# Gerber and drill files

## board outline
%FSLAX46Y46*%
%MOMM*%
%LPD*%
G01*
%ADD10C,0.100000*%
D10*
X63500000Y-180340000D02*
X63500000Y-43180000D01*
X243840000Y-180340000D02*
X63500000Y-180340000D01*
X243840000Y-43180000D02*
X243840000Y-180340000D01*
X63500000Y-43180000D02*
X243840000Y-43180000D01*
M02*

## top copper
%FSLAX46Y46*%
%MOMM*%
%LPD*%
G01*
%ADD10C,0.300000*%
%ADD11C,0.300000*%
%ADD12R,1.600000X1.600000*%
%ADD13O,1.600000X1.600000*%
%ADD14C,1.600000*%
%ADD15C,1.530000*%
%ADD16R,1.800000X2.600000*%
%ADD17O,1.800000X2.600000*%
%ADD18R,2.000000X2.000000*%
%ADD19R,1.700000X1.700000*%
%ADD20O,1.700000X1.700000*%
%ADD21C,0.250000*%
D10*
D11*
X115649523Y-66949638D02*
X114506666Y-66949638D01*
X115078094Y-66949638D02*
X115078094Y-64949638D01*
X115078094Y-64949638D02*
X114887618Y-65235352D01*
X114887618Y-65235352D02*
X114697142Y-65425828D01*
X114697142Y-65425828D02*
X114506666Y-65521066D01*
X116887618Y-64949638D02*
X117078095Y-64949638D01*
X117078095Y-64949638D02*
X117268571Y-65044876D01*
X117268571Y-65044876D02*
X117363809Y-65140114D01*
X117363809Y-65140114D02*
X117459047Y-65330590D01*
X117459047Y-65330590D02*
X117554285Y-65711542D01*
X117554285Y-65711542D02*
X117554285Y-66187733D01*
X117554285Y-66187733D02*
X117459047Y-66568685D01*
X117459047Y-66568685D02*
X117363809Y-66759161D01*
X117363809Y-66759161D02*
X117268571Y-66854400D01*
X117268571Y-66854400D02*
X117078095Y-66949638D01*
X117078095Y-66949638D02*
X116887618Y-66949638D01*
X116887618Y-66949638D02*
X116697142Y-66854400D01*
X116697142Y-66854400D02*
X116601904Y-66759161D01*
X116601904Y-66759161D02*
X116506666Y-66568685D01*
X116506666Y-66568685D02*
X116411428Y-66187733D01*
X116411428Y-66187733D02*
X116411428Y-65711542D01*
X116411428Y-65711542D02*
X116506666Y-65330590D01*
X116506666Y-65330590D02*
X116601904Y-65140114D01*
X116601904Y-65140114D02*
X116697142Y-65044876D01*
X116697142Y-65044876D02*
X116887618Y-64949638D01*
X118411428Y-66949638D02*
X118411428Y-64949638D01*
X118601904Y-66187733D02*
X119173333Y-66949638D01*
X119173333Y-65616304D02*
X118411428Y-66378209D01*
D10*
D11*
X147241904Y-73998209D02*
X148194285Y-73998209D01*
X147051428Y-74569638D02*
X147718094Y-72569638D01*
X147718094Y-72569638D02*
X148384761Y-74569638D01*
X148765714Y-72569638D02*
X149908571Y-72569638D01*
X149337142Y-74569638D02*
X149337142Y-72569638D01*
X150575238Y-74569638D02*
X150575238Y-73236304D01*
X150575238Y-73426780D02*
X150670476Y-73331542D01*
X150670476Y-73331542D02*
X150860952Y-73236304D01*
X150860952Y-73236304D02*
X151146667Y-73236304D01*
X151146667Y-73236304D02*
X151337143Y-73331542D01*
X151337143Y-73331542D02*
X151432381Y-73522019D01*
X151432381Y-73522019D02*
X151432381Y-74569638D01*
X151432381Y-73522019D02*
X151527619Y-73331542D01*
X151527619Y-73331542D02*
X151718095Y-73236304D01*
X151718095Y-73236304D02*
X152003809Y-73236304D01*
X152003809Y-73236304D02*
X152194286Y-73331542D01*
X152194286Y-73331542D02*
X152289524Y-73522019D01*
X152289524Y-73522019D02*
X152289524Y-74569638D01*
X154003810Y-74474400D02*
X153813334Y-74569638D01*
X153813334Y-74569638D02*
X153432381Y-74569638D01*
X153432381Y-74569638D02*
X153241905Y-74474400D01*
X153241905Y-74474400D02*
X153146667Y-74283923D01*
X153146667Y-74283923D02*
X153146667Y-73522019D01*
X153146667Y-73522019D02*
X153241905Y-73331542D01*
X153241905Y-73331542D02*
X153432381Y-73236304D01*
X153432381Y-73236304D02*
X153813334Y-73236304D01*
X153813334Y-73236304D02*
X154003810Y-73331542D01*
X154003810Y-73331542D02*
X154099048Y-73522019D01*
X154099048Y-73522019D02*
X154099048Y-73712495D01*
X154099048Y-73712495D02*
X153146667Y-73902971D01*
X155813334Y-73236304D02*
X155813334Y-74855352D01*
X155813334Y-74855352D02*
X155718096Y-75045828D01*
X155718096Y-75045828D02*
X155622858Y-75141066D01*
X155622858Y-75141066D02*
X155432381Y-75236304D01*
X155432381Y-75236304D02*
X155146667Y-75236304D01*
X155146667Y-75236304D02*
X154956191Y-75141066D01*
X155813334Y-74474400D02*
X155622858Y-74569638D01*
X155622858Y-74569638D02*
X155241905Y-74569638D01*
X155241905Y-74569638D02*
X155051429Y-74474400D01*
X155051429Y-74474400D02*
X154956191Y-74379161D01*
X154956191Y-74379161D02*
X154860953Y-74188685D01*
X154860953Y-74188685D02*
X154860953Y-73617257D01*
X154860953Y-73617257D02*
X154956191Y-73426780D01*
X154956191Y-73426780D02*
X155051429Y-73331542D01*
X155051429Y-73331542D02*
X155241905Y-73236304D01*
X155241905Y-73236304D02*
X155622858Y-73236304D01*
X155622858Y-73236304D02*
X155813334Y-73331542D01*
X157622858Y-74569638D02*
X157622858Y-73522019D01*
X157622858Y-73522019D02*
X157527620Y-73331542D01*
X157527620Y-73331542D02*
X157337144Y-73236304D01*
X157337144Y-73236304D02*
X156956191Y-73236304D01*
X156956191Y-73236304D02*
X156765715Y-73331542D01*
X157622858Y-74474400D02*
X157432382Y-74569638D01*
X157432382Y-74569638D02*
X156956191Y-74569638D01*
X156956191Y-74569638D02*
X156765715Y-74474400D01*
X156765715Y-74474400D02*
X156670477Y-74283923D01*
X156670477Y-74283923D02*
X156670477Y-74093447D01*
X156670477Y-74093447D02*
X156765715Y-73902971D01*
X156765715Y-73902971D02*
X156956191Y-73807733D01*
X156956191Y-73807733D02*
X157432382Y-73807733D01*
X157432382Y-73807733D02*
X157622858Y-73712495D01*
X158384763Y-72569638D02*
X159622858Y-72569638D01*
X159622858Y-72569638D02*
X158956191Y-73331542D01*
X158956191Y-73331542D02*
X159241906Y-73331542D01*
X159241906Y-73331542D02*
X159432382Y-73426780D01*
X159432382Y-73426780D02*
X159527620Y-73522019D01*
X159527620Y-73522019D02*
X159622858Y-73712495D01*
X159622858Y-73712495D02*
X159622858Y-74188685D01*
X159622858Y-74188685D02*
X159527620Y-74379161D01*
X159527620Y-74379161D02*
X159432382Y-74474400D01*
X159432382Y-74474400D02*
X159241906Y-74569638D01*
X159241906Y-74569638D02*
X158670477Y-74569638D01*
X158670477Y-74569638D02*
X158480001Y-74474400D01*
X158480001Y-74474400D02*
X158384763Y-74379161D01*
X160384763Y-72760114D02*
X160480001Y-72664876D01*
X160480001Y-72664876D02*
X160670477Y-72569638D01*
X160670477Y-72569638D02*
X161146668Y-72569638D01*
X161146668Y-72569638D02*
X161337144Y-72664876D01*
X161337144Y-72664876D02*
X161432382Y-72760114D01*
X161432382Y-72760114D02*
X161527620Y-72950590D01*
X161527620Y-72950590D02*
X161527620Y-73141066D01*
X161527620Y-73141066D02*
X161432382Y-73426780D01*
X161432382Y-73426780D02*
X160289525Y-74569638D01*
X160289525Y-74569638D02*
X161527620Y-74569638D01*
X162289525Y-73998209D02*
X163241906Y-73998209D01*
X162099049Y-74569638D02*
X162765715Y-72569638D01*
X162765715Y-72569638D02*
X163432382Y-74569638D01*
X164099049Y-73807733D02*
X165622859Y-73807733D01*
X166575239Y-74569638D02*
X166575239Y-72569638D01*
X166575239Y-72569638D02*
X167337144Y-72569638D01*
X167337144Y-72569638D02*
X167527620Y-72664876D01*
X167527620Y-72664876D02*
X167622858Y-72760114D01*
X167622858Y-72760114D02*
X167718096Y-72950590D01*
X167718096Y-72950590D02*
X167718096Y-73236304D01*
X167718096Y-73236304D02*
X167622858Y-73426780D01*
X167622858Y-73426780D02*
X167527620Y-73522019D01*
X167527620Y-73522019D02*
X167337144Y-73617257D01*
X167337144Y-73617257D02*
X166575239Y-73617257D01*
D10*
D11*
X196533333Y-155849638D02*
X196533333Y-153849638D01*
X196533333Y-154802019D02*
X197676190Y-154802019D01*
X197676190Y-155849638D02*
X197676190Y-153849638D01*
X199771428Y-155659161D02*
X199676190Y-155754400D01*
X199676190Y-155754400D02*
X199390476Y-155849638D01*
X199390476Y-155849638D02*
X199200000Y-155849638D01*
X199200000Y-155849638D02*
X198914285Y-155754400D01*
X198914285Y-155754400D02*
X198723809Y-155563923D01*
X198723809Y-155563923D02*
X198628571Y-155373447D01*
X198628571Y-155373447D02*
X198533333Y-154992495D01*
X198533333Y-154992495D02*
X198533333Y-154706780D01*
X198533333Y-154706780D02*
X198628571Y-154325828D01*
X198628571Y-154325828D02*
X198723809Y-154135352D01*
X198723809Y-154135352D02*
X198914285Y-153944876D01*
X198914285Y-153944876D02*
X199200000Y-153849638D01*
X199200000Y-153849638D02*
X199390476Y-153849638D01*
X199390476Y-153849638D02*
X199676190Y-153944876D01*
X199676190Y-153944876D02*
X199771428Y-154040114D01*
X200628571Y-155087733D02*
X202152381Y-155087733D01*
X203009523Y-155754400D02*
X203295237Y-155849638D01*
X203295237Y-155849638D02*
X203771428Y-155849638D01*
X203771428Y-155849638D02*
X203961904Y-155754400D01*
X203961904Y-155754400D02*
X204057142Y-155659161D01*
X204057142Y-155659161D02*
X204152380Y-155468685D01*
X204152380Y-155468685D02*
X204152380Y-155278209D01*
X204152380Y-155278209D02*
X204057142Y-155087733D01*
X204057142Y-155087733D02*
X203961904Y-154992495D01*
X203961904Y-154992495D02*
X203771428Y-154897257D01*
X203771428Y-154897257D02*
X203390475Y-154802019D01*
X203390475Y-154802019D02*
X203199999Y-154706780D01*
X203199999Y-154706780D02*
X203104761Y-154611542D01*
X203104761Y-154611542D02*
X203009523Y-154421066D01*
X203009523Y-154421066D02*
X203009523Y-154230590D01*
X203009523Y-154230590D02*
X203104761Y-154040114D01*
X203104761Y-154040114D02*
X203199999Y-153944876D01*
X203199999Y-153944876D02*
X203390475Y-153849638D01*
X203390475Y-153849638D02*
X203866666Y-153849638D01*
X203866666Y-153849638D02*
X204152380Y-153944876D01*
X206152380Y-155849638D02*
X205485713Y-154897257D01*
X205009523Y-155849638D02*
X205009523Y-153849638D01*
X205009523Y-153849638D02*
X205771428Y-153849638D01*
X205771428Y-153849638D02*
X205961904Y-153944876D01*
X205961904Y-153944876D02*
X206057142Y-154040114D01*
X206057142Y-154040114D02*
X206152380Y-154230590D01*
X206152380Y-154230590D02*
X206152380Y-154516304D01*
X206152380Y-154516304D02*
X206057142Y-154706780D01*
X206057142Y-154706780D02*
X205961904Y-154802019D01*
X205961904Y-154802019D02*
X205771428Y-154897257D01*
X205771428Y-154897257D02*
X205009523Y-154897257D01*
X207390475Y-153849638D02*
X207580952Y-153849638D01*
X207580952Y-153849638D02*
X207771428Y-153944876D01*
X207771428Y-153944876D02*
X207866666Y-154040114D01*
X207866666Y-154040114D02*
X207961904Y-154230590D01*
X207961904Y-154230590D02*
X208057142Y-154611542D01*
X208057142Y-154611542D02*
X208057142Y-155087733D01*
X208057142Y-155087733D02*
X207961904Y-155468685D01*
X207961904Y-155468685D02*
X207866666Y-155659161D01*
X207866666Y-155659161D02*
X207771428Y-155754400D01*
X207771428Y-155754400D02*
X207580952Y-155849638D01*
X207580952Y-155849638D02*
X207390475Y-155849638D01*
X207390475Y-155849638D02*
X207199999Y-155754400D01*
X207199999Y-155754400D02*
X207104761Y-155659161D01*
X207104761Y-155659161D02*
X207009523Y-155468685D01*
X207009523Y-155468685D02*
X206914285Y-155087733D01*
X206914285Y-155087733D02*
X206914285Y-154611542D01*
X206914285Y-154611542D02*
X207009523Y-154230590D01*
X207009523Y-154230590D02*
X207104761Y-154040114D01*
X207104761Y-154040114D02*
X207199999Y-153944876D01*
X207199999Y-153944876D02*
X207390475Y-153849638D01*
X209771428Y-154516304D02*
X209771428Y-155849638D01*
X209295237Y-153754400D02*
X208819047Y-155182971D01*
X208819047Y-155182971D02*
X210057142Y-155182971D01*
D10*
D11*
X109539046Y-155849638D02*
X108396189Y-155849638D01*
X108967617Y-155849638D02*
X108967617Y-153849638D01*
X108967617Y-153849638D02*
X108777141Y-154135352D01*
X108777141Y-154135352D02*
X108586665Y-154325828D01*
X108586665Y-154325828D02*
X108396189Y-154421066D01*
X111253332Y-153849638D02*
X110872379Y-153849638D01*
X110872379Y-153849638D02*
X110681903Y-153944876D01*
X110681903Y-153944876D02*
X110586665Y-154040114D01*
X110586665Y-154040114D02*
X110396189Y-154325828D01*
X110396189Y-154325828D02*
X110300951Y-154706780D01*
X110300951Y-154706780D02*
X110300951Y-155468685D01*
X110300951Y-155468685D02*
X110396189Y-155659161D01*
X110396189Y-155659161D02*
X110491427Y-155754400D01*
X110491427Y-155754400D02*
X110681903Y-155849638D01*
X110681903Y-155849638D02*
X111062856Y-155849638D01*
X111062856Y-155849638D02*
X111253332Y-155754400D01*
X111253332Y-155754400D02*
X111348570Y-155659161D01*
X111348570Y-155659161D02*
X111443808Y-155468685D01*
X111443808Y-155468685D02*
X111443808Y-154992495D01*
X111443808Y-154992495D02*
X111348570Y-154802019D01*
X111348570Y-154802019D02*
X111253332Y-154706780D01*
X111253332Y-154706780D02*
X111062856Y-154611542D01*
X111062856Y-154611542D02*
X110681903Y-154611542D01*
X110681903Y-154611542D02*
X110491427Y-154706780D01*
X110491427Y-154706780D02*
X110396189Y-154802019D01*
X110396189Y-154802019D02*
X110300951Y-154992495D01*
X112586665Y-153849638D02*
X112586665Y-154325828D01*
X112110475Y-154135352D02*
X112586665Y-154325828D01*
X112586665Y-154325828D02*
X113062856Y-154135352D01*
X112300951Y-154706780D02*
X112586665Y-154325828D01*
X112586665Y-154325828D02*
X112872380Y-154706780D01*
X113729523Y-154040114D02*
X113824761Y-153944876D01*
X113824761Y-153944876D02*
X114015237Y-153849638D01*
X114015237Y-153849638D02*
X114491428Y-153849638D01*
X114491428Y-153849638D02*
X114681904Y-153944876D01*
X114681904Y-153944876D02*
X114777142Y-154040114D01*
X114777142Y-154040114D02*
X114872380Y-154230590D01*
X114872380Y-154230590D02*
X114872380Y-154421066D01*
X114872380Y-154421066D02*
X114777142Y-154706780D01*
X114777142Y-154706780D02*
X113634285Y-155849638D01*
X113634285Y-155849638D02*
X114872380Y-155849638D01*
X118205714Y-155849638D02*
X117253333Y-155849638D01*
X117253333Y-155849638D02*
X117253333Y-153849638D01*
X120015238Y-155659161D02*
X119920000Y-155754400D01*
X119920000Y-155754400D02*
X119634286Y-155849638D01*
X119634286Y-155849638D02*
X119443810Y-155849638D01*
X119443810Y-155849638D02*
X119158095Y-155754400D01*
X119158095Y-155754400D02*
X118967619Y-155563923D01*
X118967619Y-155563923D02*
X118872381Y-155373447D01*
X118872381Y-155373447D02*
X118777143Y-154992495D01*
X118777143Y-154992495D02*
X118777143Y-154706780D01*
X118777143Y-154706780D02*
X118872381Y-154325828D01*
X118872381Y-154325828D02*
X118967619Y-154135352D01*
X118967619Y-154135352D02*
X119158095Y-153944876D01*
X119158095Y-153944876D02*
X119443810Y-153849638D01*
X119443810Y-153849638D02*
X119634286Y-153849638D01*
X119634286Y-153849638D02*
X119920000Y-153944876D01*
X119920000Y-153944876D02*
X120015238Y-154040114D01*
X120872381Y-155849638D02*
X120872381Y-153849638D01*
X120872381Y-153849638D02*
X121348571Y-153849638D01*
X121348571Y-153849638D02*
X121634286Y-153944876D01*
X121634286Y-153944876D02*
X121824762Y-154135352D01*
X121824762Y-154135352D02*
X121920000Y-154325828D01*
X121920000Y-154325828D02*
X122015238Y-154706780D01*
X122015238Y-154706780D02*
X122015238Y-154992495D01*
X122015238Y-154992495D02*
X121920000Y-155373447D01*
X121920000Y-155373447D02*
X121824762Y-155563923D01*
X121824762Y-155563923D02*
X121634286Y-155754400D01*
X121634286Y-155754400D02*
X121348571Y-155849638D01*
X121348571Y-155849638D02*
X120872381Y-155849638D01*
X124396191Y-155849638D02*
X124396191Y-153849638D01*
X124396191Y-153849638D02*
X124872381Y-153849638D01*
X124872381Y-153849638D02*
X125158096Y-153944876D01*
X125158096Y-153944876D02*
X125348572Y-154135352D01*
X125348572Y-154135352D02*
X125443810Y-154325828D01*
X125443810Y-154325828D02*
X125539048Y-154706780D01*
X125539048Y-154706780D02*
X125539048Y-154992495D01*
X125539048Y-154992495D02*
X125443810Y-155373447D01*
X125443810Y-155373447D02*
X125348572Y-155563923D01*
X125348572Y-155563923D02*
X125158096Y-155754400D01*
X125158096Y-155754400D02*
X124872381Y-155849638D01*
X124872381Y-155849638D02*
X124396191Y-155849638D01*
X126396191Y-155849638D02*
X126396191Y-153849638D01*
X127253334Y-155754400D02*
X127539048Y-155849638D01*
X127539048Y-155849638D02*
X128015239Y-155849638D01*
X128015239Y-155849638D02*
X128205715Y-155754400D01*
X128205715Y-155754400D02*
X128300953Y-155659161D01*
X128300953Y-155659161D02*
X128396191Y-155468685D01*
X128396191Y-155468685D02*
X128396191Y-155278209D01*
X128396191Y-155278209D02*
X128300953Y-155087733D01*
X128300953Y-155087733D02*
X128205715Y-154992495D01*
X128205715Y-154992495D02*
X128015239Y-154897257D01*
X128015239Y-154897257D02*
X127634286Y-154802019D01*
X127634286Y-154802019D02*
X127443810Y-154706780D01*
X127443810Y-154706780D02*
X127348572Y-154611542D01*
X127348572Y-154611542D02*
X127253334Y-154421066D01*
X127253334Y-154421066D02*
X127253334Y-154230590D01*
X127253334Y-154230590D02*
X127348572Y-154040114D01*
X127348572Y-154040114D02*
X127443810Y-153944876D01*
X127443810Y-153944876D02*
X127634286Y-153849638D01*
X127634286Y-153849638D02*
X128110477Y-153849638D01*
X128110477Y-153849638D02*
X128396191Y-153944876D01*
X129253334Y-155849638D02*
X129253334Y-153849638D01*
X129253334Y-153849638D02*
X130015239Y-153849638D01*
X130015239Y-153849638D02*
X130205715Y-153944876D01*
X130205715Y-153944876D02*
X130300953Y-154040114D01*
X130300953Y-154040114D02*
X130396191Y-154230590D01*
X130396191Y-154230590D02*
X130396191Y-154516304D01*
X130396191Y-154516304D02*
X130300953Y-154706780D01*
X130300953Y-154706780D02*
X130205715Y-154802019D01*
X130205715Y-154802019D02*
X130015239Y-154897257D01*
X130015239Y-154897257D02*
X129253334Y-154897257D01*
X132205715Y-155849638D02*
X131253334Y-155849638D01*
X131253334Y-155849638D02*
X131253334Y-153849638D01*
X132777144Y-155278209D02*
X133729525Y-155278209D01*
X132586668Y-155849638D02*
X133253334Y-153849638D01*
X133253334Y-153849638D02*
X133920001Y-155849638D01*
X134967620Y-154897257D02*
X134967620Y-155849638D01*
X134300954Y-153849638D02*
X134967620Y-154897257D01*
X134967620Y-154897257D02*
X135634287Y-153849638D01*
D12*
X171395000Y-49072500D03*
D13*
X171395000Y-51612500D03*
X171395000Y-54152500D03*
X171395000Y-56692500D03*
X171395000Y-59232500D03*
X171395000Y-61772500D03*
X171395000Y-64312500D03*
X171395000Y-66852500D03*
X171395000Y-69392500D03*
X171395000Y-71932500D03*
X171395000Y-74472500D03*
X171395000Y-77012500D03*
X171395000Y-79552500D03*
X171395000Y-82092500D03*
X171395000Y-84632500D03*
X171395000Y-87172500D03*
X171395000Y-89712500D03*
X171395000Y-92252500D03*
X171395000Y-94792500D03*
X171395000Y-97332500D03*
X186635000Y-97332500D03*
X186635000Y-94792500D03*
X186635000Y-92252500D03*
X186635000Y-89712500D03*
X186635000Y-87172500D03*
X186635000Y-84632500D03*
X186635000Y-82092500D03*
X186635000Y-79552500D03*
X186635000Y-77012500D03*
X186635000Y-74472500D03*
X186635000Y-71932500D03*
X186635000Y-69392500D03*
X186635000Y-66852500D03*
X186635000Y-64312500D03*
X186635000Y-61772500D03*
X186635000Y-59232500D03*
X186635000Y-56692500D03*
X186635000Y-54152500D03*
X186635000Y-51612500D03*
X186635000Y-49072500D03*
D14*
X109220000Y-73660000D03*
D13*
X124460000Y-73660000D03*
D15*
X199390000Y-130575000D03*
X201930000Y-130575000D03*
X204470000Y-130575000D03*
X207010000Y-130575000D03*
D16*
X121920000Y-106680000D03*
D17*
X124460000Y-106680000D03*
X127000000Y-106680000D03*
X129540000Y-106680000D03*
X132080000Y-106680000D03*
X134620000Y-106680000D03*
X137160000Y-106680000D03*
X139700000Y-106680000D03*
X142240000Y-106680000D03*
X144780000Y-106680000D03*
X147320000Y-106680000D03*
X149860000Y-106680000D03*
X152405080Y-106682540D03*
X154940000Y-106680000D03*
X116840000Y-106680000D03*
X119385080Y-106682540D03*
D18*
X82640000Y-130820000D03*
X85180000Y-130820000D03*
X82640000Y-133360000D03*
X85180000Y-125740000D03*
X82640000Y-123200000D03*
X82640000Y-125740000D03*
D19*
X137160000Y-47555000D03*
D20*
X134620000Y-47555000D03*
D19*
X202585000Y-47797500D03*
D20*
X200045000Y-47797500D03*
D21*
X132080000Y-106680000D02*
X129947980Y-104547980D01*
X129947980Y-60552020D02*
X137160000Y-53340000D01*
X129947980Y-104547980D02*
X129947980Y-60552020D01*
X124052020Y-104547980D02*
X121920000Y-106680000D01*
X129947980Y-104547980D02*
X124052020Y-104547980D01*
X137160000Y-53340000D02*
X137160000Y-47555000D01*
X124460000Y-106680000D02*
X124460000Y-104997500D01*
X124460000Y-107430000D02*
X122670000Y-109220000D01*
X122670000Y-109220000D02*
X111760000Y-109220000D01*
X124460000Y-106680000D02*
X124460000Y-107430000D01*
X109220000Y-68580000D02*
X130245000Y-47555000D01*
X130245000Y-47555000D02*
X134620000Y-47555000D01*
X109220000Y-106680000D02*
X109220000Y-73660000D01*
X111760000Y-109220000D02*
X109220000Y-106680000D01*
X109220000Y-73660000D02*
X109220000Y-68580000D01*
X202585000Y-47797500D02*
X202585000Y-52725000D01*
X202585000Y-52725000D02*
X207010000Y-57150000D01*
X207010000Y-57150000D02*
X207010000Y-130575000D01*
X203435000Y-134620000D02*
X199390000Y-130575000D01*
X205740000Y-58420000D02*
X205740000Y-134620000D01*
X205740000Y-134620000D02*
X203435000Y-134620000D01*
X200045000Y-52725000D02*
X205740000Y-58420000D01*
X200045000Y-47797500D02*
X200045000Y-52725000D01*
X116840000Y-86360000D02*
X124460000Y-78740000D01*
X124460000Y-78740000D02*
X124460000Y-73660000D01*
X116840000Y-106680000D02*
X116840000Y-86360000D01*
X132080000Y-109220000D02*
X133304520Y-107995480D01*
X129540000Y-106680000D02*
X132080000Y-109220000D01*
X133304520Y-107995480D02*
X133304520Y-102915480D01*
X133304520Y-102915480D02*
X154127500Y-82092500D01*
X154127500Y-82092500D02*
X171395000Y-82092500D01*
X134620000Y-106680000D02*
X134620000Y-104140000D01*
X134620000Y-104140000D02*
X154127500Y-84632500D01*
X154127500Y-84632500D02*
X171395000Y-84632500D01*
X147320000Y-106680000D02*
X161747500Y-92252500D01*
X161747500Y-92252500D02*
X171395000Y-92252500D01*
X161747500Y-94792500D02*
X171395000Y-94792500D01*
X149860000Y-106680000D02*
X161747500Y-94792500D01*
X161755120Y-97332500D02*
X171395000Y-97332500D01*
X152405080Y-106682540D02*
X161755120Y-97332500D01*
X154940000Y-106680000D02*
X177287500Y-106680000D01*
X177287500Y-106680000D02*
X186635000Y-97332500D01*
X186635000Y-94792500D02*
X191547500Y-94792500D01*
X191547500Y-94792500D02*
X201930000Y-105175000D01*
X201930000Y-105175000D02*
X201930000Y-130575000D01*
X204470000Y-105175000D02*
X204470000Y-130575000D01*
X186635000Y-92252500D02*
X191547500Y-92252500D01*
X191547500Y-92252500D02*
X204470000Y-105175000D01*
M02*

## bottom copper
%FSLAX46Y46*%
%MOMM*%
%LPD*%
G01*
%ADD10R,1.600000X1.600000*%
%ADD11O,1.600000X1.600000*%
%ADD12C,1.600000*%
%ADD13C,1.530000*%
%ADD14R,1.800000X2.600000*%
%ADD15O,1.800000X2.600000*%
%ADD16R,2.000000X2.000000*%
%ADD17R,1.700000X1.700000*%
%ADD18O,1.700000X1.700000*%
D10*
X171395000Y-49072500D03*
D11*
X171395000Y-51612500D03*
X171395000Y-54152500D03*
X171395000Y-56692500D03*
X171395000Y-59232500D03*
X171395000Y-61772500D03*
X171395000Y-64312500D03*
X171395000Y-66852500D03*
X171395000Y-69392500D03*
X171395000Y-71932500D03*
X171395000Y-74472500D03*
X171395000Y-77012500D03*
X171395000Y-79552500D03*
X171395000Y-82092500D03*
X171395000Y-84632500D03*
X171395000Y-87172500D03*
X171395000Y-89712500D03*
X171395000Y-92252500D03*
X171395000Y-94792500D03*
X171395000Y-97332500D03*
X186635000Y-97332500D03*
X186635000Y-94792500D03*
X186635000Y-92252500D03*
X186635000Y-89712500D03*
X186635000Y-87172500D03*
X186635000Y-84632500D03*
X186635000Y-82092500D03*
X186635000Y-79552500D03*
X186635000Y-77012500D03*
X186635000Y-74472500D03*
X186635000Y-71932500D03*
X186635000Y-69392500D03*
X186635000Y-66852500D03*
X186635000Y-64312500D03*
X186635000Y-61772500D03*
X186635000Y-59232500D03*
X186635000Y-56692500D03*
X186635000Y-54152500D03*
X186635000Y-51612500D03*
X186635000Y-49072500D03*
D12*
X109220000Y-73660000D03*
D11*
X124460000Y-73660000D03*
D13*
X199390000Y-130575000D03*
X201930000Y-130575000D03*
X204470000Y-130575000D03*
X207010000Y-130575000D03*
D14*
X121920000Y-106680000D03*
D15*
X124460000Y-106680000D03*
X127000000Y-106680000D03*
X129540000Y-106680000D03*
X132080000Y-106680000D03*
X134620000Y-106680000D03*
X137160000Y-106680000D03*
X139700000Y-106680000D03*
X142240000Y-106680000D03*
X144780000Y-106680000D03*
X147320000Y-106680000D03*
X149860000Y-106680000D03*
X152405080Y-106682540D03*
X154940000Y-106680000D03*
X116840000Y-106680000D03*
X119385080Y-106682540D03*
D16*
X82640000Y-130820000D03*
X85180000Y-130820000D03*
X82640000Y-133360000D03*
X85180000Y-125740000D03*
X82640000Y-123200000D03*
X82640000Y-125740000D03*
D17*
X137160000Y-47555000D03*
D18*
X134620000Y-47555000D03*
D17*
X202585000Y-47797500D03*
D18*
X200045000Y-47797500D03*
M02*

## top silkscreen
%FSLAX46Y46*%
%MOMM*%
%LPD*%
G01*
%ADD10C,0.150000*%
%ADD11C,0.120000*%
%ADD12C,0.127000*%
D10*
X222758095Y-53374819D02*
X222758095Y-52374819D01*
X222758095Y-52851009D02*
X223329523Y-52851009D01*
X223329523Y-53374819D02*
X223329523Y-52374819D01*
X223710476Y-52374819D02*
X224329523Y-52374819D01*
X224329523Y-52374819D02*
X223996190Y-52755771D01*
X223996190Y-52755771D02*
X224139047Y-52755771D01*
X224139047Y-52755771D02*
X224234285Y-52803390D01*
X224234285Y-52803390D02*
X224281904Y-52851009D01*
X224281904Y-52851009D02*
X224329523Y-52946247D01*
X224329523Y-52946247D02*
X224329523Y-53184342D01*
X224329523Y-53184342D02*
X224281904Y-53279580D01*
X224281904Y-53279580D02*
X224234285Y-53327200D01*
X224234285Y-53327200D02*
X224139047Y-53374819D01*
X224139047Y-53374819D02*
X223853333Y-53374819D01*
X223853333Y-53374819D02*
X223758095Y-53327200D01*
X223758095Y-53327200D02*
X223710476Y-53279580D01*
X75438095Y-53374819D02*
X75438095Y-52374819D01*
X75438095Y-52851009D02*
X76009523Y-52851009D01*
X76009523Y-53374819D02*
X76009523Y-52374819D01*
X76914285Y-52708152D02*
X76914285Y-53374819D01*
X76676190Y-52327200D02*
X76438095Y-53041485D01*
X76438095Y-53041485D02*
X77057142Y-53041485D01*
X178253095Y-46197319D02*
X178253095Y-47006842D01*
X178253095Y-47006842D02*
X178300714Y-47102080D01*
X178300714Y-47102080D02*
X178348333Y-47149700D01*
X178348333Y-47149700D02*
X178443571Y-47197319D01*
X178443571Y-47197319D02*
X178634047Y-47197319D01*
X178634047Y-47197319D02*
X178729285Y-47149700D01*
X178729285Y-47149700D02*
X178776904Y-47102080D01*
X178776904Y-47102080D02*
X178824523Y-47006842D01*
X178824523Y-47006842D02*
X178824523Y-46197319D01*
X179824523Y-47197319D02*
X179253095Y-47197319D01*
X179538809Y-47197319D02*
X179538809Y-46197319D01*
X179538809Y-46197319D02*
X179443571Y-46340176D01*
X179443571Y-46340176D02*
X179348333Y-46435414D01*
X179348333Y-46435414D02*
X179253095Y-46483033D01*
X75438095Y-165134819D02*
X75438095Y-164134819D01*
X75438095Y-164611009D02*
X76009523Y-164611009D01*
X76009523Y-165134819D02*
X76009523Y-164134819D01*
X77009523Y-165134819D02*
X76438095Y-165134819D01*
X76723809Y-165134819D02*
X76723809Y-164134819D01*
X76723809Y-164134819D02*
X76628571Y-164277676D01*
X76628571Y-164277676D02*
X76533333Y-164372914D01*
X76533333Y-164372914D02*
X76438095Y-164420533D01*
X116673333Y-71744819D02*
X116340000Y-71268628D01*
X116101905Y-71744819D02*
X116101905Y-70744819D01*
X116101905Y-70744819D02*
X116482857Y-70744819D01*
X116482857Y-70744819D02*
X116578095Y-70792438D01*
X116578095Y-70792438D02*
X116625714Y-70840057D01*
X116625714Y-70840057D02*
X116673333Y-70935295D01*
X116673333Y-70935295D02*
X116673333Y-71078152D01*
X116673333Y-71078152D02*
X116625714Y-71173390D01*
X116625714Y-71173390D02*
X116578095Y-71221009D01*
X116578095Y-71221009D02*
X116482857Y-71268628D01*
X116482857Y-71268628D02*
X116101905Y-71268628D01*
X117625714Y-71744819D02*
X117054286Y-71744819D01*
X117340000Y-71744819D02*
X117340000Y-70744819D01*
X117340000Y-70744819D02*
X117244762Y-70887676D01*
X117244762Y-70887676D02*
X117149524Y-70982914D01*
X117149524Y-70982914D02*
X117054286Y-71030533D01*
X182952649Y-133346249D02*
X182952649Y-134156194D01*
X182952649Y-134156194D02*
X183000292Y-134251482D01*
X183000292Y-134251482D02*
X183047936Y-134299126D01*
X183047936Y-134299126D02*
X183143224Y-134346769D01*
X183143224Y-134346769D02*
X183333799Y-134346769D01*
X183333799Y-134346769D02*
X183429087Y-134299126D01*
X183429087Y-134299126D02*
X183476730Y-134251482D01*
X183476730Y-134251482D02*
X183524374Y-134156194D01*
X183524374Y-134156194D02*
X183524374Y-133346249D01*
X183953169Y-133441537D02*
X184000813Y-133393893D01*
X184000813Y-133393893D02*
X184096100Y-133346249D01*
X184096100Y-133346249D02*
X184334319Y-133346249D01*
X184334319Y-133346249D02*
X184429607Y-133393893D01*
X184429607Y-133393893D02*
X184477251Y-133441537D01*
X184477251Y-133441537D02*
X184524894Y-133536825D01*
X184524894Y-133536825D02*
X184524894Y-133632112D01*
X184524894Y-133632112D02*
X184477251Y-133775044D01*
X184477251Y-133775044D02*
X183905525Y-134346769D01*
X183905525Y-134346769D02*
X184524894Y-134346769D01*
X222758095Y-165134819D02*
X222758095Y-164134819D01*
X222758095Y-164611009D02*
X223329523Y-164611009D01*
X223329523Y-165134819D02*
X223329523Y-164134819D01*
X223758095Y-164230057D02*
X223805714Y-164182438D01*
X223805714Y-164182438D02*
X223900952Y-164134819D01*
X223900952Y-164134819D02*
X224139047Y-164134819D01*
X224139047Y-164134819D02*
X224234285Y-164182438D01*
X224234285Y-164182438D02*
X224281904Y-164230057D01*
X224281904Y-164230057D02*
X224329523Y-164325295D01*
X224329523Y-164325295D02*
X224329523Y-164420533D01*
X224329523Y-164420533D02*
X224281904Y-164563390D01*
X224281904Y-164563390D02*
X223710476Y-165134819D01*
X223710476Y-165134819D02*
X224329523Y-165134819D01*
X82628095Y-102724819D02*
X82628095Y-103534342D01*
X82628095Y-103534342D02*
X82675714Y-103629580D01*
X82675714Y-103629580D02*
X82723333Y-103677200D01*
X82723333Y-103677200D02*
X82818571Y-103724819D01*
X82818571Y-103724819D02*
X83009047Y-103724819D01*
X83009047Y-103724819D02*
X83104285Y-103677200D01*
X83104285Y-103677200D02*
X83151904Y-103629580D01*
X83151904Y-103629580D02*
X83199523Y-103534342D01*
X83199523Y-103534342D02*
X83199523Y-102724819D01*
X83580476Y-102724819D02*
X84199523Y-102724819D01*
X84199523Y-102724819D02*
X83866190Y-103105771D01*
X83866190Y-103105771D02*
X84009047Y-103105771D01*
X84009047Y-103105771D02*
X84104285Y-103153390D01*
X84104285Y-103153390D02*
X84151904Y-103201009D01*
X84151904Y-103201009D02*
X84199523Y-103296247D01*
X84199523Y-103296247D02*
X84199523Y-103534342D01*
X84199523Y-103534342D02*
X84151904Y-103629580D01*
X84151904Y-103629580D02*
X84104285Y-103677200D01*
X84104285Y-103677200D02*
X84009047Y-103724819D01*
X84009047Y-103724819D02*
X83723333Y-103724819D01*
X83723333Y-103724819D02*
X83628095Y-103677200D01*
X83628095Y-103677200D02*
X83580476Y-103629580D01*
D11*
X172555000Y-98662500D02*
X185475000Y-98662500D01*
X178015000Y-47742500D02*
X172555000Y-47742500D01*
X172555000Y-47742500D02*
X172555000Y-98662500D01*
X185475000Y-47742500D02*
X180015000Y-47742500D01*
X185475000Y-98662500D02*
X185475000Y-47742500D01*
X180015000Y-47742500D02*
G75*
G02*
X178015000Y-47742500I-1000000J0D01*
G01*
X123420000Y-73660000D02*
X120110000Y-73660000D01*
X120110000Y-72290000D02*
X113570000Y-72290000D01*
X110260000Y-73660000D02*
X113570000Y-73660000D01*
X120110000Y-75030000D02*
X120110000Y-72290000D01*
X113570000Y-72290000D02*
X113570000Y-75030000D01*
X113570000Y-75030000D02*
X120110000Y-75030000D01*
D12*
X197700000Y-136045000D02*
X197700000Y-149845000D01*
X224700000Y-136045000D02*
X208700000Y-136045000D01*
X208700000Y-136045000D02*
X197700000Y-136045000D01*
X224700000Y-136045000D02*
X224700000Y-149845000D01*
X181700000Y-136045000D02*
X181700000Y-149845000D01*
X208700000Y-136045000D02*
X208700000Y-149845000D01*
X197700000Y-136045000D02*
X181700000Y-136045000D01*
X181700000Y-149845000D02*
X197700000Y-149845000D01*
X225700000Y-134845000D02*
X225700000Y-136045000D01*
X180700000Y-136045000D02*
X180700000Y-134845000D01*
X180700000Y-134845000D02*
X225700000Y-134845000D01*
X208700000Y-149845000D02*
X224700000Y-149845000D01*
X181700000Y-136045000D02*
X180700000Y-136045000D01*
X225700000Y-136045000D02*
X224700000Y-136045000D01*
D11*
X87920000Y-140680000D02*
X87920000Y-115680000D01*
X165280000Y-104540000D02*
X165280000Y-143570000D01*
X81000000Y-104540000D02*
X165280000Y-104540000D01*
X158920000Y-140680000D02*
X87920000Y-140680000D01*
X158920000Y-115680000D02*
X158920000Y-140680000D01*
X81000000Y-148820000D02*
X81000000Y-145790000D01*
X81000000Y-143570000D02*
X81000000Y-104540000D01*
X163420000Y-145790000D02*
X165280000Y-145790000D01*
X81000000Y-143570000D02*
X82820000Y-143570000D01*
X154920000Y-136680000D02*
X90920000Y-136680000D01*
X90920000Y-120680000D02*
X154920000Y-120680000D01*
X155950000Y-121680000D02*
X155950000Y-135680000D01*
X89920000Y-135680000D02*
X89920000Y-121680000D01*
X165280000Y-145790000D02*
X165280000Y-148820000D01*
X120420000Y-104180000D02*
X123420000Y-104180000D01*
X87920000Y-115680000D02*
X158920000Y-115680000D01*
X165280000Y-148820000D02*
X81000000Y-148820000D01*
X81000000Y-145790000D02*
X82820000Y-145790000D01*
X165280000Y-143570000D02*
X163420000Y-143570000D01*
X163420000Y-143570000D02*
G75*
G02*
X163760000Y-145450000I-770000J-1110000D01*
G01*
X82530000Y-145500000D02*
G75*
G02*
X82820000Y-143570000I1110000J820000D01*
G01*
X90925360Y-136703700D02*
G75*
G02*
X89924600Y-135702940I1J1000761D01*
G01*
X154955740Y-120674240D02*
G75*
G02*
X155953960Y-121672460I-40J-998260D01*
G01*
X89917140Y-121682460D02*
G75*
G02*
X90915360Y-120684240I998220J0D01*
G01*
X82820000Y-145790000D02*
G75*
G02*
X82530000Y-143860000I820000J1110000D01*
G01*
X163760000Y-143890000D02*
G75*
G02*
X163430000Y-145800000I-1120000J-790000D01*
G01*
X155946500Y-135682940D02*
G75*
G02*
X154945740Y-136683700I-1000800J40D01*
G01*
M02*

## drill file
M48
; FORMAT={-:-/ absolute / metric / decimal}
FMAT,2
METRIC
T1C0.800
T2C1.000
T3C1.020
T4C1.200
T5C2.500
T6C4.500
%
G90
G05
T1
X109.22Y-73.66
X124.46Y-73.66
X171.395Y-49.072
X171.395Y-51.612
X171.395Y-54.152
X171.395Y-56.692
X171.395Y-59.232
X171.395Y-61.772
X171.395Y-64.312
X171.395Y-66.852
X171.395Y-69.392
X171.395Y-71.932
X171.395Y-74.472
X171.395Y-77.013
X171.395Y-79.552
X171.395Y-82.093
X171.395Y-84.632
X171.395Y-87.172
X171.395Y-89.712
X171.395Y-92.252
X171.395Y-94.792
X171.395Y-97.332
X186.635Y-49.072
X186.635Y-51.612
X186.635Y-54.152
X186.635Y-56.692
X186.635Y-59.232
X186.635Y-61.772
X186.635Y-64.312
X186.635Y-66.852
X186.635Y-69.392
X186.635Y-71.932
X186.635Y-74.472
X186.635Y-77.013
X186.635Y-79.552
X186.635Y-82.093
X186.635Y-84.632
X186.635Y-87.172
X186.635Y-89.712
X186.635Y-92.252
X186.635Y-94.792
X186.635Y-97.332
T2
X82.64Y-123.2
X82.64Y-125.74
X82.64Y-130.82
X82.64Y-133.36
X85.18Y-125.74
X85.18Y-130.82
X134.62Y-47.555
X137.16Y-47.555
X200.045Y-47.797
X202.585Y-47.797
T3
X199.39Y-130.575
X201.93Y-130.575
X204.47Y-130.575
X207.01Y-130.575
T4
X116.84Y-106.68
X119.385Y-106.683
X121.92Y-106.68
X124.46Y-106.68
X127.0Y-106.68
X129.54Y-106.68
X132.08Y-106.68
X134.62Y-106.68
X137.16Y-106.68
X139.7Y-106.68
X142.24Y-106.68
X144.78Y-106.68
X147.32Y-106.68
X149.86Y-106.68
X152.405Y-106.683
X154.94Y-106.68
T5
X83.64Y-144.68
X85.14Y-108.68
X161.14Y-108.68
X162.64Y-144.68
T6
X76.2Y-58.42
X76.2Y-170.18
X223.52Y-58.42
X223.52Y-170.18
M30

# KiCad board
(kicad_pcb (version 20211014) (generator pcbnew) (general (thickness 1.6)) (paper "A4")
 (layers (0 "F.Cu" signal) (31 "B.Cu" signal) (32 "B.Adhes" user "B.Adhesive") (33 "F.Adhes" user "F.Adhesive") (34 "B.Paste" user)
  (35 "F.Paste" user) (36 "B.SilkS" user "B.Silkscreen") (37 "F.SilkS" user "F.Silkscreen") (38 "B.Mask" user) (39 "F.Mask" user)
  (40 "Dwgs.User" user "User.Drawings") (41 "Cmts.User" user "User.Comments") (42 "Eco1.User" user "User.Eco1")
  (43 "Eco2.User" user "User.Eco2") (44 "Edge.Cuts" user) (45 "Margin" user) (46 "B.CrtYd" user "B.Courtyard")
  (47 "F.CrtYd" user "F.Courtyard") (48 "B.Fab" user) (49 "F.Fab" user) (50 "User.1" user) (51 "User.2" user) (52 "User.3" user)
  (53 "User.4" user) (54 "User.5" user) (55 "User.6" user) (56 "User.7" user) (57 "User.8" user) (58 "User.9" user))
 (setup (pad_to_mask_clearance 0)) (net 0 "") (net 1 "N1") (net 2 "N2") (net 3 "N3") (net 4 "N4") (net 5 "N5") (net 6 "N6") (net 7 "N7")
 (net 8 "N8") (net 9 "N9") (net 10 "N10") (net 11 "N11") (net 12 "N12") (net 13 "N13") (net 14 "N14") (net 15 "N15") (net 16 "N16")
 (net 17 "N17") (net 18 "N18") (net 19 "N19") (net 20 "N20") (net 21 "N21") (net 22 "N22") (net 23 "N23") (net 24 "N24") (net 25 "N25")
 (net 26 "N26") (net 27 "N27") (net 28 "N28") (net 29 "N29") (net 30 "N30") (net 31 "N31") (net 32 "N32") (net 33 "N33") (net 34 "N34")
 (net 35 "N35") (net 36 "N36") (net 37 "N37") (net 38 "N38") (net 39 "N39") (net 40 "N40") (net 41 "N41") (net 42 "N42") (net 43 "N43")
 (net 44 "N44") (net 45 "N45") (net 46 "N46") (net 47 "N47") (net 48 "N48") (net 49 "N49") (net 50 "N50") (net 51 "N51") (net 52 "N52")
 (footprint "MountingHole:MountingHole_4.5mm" (layer "F.Cu") (at 223.52 58.42)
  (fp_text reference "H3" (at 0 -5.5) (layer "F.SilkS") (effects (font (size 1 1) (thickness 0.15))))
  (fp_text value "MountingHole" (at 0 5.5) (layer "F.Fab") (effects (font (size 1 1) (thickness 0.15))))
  (pad "" np_thru_hole circle (at 0 0) (size 4.5 4.5) (drill 4.5) (layers *.Cu *.Mask)))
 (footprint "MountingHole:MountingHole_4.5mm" (layer "F.Cu") (at 76.2 58.42)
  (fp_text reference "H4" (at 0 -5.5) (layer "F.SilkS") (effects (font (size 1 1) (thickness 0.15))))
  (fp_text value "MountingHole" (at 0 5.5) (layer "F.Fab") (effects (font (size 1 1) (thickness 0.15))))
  (pad "" np_thru_hole circle (at 0 0) (size 4.5 4.5) (drill 4.5) (layers *.Cu *.Mask)))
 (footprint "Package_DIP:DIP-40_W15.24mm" (layer "F.Cu") (at 171.395 49.0725)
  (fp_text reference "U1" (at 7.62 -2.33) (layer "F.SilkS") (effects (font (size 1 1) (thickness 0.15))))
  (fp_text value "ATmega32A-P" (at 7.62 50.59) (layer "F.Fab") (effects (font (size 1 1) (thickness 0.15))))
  (fp_line (start 1.16 49.59) (end 14.08 49.59) (layer "F.SilkS") (width 0.12))
  (fp_line (start 6.62 -1.33) (end 1.16 -1.33) (layer "F.SilkS") (width 0.12))
  (fp_line (start 1.16 -1.33) (end 1.16 49.59) (layer "F.SilkS") (width 0.12))
  (fp_line (start 14.08 -1.33) (end 8.62 -1.33) (layer "F.SilkS") (width 0.12))
  (fp_line (start 14.08 49.59) (end 14.08 -1.33) (layer "F.SilkS") (width 0.12))
  (fp_arc (start 8.62 -1.33) (mid 7.62 -0.33) (end 6.62 -1.33) (layer "F.SilkS") (width 0.12))
  (pad "1" thru_hole rect (at 0 0) (size 1.6 1.6) (drill 0.8) (layers *.Cu *.Mask) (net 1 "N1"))
  (pad "2" thru_hole oval (at 0 2.54) (size 1.6 1.6) (drill 0.8) (layers *.Cu *.Mask) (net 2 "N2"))
  (pad "3" thru_hole oval (at 0 5.08) (size 1.6 1.6) (drill 0.8) (layers *.Cu *.Mask) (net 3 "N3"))
  (pad "4" thru_hole oval (at 0 7.62) (size 1.6 1.6) (drill 0.8) (layers *.Cu *.Mask) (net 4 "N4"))
  (pad "5" thru_hole oval (at 0 10.16) (size 1.6 1.6) (drill 0.8) (layers *.Cu *.Mask) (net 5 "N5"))
  (pad "6" thru_hole oval (at 0 12.7) (size 1.6 1.6) (drill 0.8) (layers *.Cu *.Mask) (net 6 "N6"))
  (pad "7" thru_hole oval (at 0 15.24) (size 1.6 1.6) (drill 0.8) (layers *.Cu *.Mask) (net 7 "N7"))
  (pad "8" thru_hole oval (at 0 17.78) (size 1.6 1.6) (drill 0.8) (layers *.Cu *.Mask) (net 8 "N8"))
  (pad "9" thru_hole oval (at 0 20.32) (size 1.6 1.6) (drill 0.8) (layers *.Cu *.Mask) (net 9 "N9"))
  (pad "10" thru_hole oval (at 0 22.86) (size 1.6 1.6) (drill 0.8) (layers *.Cu *.Mask) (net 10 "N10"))
  (pad "11" thru_hole oval (at 0 25.4) (size 1.6 1.6) (drill 0.8) (layers *.Cu *.Mask) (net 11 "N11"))
  (pad "12" thru_hole oval (at 0 27.94) (size 1.6 1.6) (drill 0.8) (layers *.Cu *.Mask) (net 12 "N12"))
  (pad "13" thru_hole oval (at 0 30.48) (size 1.6 1.6) (drill 0.8) (layers *.Cu *.Mask) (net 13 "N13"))
  (pad "14" thru_hole oval (at 0 33.02) (size 1.6 1.6) (drill 0.8) (layers *.Cu *.Mask) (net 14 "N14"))
  (pad "15" thru_hole oval (at 0 35.56) (size 1.6 1.6) (drill 0.8) (layers *.Cu *.Mask) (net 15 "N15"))
  (pad "16" thru_hole oval (at 0 38.1) (size 1.6 1.6) (drill 0.8) (layers *.Cu *.Mask) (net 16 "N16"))
  (pad "17" thru_hole oval (at 0 40.64) (size 1.6 1.6) (drill 0.8) (layers *.Cu *.Mask) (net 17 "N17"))
  (pad "18" thru_hole oval (at 0 43.18) (size 1.6 1.6) (drill 0.8) (layers *.Cu *.Mask) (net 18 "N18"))
  (pad "19" thru_hole oval (at 0 45.72) (size 1.6 1.6) (drill 0.8) (layers *.Cu *.Mask) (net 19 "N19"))
  (pad "20" thru_hole oval (at 0 48.26) (size 1.6 1.6) (drill 0.8) (layers *.Cu *.Mask) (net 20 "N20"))
  (pad "21" thru_hole oval (at 15.24 48.26) (size 1.6 1.6) (drill 0.8) (layers *.Cu *.Mask) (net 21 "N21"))
  (pad "22" thru_hole oval (at 15.24 45.72) (size 1.6 1.6) (drill 0.8) (layers *.Cu *.Mask) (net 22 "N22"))
  (pad "23" thru_hole oval (at 15.24 43.18) (size 1.6 1.6) (drill 0.8) (layers *.Cu *.Mask) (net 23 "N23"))
  (pad "24" thru_hole oval (at 15.24 40.64) (size 1.6 1.6) (drill 0.8) (layers *.Cu *.Mask) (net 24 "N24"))
  (pad "25" thru_hole oval (at 15.24 38.1) (size 1.6 1.6) (drill 0.8) (layers *.Cu *.Mask) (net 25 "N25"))
  (pad "26" thru_hole oval (at 15.24 35.56) (size 1.6 1.6) (drill 0.8) (layers *.Cu *.Mask) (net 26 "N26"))
  (pad "27" thru_hole oval (at 15.24 33.02) (size 1.6 1.6) (drill 0.8) (layers *.Cu *.Mask) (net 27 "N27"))
  (pad "28" thru_hole oval (at 15.24 30.48) (size 1.6 1.6) (drill 0.8) (layers *.Cu *.Mask) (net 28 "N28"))
  (pad "29" thru_hole oval (at 15.24 27.94) (size 1.6 1.6) (drill 0.8) (layers *.Cu *.Mask) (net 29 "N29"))
  (pad "30" thru_hole oval (at 15.24 25.4) (size 1.6 1.6) (drill 0.8) (layers *.Cu *.Mask) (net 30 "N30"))
  (pad "31" thru_hole oval (at 15.24 22.86) (size 1.6 1.6) (drill 0.8) (layers *.Cu *.Mask) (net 11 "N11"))
  (pad "32" thru_hole oval (at 15.24 20.32) (size 1.6 1.6) (drill 0.8) (layers *.Cu *.Mask) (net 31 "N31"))
  (pad "33" thru_hole oval (at 15.24 17.78) (size 1.6 1.6) (drill 0.8) (layers *.Cu *.Mask) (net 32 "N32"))
  (pad "34" thru_hole oval (at 15.24 15.24) (size 1.6 1.6) (drill 0.8) (layers *.Cu *.Mask) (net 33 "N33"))
  (pad "35" thru_hole oval (at 15.24 12.7) (size 1.6 1.6) (drill 0.8) (layers *.Cu *.Mask) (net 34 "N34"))
  (pad "36" thru_hole oval (at 15.24 10.16) (size 1.6 1.6) (drill 0.8) (layers *.Cu *.Mask) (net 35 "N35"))
  (pad "37" thru_hole oval (at 15.24 7.62) (size 1.6 1.6) (drill 0.8) (layers *.Cu *.Mask) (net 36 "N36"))
  (pad "38" thru_hole oval (at 15.24 5.08) (size 1.6 1.6) (drill 0.8) (layers *.Cu *.Mask) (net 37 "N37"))
  (pad "39" thru_hole oval (at 15.24 2.54) (size 1.6 1.6) (drill 0.8) (layers *.Cu *.Mask) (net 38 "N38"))
  (pad "40" thru_hole oval (at 15.24 0) (size 1.6 1.6) (drill 0.8) (layers *.Cu *.Mask) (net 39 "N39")))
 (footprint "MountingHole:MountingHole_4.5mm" (layer "F.Cu") (at 76.2 170.18)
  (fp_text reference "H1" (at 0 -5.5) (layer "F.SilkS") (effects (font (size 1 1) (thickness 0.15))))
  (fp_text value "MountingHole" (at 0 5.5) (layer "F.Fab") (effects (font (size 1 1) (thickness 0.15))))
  (pad "" np_thru_hole circle (at 0 0) (size 4.5 4.5) (drill 4.5) (layers *.Cu *.Mask)))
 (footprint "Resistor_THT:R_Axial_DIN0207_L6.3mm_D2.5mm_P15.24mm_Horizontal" (layer "F.Cu") (at 109.22 73.66)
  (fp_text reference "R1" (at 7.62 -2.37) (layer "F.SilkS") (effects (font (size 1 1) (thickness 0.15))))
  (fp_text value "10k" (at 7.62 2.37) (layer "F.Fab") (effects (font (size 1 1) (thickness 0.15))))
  (fp_line (start 14.2 0) (end 10.89 0) (layer "F.SilkS") (width 0.12))
  (fp_line (start 10.89 -1.37) (end 4.35 -1.37) (layer "F.SilkS") (width 0.12))
  (fp_line (start 1.04 0) (end 4.35 0) (layer "F.SilkS") (width 0.12))
  (fp_line (start 10.89 1.37) (end 10.89 -1.37) (layer "F.SilkS") (width 0.12))
  (fp_line (start 4.35 -1.37) (end 4.35 1.37) (layer "F.SilkS") (width 0.12))
  (fp_line (start 4.35 1.37) (end 10.89 1.37) (layer "F.SilkS") (width 0.12))
  (pad "1" thru_hole circle (at 0 0) (size 1.6 1.6) (drill 0.8) (layers *.Cu *.Mask) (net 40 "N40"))
  (pad "2" thru_hole oval (at 15.24 0) (size 1.6 1.6) (drill 0.8) (layers *.Cu *.Mask) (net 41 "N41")))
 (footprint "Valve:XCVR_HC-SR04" (layer "F.Cu") (at 203.2 130.575)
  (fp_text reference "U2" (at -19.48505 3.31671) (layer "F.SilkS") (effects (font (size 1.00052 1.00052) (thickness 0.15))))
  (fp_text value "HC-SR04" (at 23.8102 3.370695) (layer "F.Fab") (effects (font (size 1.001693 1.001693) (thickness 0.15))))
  (fp_line (start -5.5 5.47) (end -5.5 19.27) (layer "F.SilkS") (width 0.127))
  (fp_line (start 21.5 5.47) (end 5.5 5.47) (layer "F.SilkS") (width 0.127))
  (fp_line (start 5.5 5.47) (end -5.5 5.47) (layer "F.SilkS") (width 0.127))
  (fp_line (start 21.5 5.47) (end 21.5 19.27) (layer "F.SilkS") (width 0.127))
  (fp_line (start -21.5 5.47) (end -21.5 19.27) (layer "F.SilkS") (width 0.127))
  (fp_line (start 5.5 5.47) (end 5.5 19.27) (layer "F.SilkS") (width 0.127))
  (fp_line (start -5.5 5.47) (end -21.5 5.47) (layer "F.SilkS") (width 0.127))
  (fp_line (start -21.5 19.27) (end -5.5 19.27) (layer "F.SilkS") (width 0.127))
  (fp_line (start 22.5 4.27) (end 22.5 5.47) (layer "F.SilkS") (width 0.127))
  (fp_line (start -22.5 5.47) (end -22.5 4.27) (layer "F.SilkS") (width 0.127))
  (fp_line (start -22.5 4.27) (end 22.5 4.27) (layer "F.SilkS") (width 0.127))
  (fp_line (start 5.5 19.27) (end 21.5 19.27) (layer "F.SilkS") (width 0.127))
  (fp_line (start -21.5 5.47) (end -22.5 5.47) (layer "F.SilkS") (width 0.127))
  (fp_line (start 22.5 5.47) (end 21.5 5.47) (layer "F.SilkS") (width 0.127))
  (pad "1" thru_hole circle (at -3.81 0) (size 1.53 1.53) (drill 1.02) (layers *.Cu *.Mask) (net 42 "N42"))
  (pad "2" thru_hole circle (at -1.27 0) (size 1.53 1.53) (drill 1.02) (layers *.Cu *.Mask) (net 22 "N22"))
  (pad "3" thru_hole circle (at 1.27 0) (size 1.53 1.53) (drill 1.02) (layers *.Cu *.Mask) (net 23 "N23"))
  (pad "4" thru_hole circle (at 3.81 0) (size 1.53 1.53) (drill 1.02) (layers *.Cu *.Mask) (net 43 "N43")))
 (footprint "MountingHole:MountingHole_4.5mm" (layer "F.Cu") (at 223.52 170.18)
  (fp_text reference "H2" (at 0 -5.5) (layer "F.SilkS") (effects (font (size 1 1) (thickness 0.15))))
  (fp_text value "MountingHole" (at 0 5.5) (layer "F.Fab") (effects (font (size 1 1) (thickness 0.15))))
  (pad "" np_thru_hole circle (at 0 0) (size 4.5 4.5) (drill 4.5) (layers *.Cu *.Mask)))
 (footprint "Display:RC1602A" (layer "F.Cu") (at 121.92 106.68)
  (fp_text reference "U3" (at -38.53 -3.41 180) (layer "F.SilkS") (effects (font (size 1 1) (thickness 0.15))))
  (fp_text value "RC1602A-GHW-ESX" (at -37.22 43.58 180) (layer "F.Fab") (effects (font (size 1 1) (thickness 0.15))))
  (fp_line (start -34 34) (end -34 9) (layer "F.SilkS") (width 0.12))
  (fp_line (start 43.36 -2.14) (end 43.36 36.89) (layer "F.SilkS") (width 0.12))
  (fp_line (start -40.92 -2.14) (end 43.36 -2.14) (layer "F.SilkS") (width 0.12))
  (fp_line (start 37 34) (end -34 34) (layer "F.SilkS") (width 0.12))
  (fp_line (start 37 9) (end 37 34) (layer "F.SilkS") (width 0.12))
  (fp_line (start -40.92 42.14) (end -40.92 39.11) (layer "F.SilkS") (width 0.12))
  (fp_line (start -40.92 36.89) (end -40.92 -2.14) (layer "F.SilkS") (width 0.12))
  (fp_line (start 41.5 39.11) (end 43.36 39.11) (layer "F.SilkS") (width 0.12))
  (fp_line (start -40.92 36.89) (end -39.1 36.89) (layer "F.SilkS") (width 0.12))
  (fp_line (start 33 30) (end -31 30) (layer "F.SilkS") (width 0.12))
  (fp_line (start -31 14) (end 33 14) (layer "F.SilkS") (width 0.12))
  (fp_line (start 34.03 15) (end 34.03 29) (layer "F.SilkS") (width 0.12))
  (fp_line (start -32 29) (end -32 15) (layer "F.SilkS") (width 0.12))
  (fp_line (start 43.36 39.11) (end 43.36 42.14) (layer "F.SilkS") (width 0.12))
  (fp_line (start -1.5 -2.5) (end 1.5 -2.5) (layer "F.SilkS") (width 0.12))
  (fp_line (start -34 9) (end 37 9) (layer "F.SilkS") (width 0.12))
  (fp_line (start 43.36 42.14) (end -40.92 42.14) (layer "F.SilkS") (width 0.12))
  (fp_line (start -40.92 39.11) (end -39.1 39.11) (layer "F.SilkS") (width 0.12))
  (fp_line (start 43.36 36.89) (end 41.5 36.89) (layer "F.SilkS") (width 0.12))
  (fp_arc (start 41.5 36.89) (mid 42.059361 37.759584) (end 41.84 38.77) (layer "F.SilkS") (width 0.12))
  (fp_arc (start -39.39 38.82) (mid -39.644716 37.794939) (end -39.1 36.89) (layer "F.SilkS") (width 0.12))
  (fp_arc (start -30.99464 30.0237) (mid -31.702284 29.730584) (end -31.9954 29.02294) (layer "F.SilkS") (width 0.12))
  (fp_arc (start 33.03574 13.99424) (mid 33.741576 14.286624) (end 34.03396 14.99246) (layer "F.SilkS") (width 0.12))
  (fp_arc (start -32.00286 15.00246) (mid -31.710488 14.296612) (end -31.00464 14.00424) (layer "F.SilkS") (width 0.12))
  (fp_arc (start -39.1 39.11) (mid -39.644716 38.205061) (end -39.39 37.18) (layer "F.SilkS") (width 0.12))
  (fp_arc (start 41.84 37.21) (mid 42.070574 38.233345) (end 41.51 39.12) (layer "F.SilkS") (width 0.12))
  (fp_arc (start 34.0265 29.00294) (mid 33.733372 29.710572) (end 33.02574 30.0037) (layer "F.SilkS") (width 0.12))
  (pad "" np_thru_hole circle (at -36.78 2 180) (size 2.5 2.5) (drill 2.5) (layers *.Cu *.Mask))
  (pad "" np_thru_hole circle (at -38.28 38 180) (size 2.5 2.5) (drill 2.5) (layers *.Cu *.Mask))
  (pad "" np_thru_hole circle (at 39.22 2 180) (size 2.5 2.5) (drill 2.5) (layers *.Cu *.Mask))
  (pad "" np_thru_hole circle (at 40.72 38 180) (size 2.5 2.5) (drill 2.5) (layers *.Cu *.Mask))
  (pad "1" thru_hole rect (at 0 0 180) (size 1.8 2.6) (drill 1.2) (layers *.Cu *.Mask) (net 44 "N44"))
  (pad "2" thru_hole oval (at 2.54 0 180) (size 1.8 2.6) (drill 1.2) (layers *.Cu *.Mask) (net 40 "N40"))
  (pad "3" thru_hole oval (at 5.08 0 180) (size 1.8 2.6) (drill 1.2) (layers *.Cu *.Mask) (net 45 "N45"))
  (pad "4" thru_hole oval (at 7.62 0 180) (size 1.8 2.6) (drill 1.2) (layers *.Cu *.Mask) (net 14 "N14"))
  (pad "5" thru_hole oval (at 10.16 0 180) (size 1.8 2.6) (drill 1.2) (layers *.Cu *.Mask) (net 44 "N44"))
  (pad "6" thru_hole oval (at 12.7 0 180) (size 1.8 2.6) (drill 1.2) (layers *.Cu *.Mask) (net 15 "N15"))
  (pad "7" thru_hole oval (at 15.24 0 180) (size 1.8 2.6) (drill 1.2) (layers *.Cu *.Mask) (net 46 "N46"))
  (pad "8" thru_hole oval (at 17.78 0 180) (size 1.8 2.6) (drill 1.2) (layers *.Cu *.Mask) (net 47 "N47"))
  (pad "9" thru_hole oval (at 20.32 0 180) (size 1.8 2.6) (drill 1.2) (layers *.Cu *.Mask) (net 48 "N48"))
  (pad "10" thru_hole oval (at 22.86 0 180) (size 1.8 2.6) (drill 1.2) (layers *.Cu *.Mask) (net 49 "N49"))
  (pad "11" thru_hole oval (at 25.4 0 180) (size 1.8 2.6) (drill 1.2) (layers *.Cu *.Mask) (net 18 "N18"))
  (pad "12" thru_hole oval (at 27.94 0 180) (size 1.8 2.6) (drill 1.2) (layers *.Cu *.Mask) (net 19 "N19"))
  (pad "13" thru_hole oval (at 30.48508 0.00254 180) (size 1.8 2.6) (drill 1.2) (layers *.Cu *.Mask) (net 20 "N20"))
  (pad "14" thru_hole oval (at 33.02 0 180) (size 1.8 2.6) (drill 1.2) (layers *.Cu *.Mask) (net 21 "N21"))
  (pad "15" thru_hole oval (at -5.08 0 180) (size 1.8 2.6) (drill 1.2) (layers *.Cu *.Mask) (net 41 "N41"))
  (pad "16" thru_hole oval (at -2.53492 0.00254 180) (size 1.8 2.6) (drill 1.2) (layers *.Cu *.Mask) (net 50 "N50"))
  (pad "A1" thru_hole rect (at -39.28 24.14 180) (size 2 2) (drill 1) (layers *.Cu *.Mask) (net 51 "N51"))
  (pad "A1" thru_hole rect (at -36.74 24.14 180) (size 2 2) (drill 1) (layers *.Cu *.Mask) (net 51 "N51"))
  (pad "A1" thru_hole rect (at -39.28 26.68 180) (size 2 2) (drill 1) (layers *.Cu *.Mask) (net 51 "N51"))
  (pad "K1" thru_hole rect (at -36.74 19.06 180) (size 2 2) (drill 1) (layers *.Cu *.Mask) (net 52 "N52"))
  (pad "K1" thru_hole rect (at -39.28 16.52 180) (size 2 2) (drill 1) (layers *.Cu *.Mask) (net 52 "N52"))
  (pad "K1" thru_hole rect (at -39.28 19.06 180) (size 2 2) (drill 1) (layers *.Cu *.Mask) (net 52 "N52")))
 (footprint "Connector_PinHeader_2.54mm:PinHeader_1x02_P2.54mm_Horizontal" (layer "B.Cu") (at 137.16 47.555 90)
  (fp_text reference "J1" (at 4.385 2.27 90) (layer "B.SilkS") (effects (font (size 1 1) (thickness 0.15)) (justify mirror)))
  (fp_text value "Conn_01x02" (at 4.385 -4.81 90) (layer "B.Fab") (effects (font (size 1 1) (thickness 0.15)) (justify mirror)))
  (pad "1" thru_hole rect (at 0 0 90) (size 1.7 1.7) (drill 1) (layers *.Cu *.Mask) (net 44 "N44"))
  (pad "2" thru_hole oval (at 0 -2.54 90) (size 1.7 1.7) (drill 1) (layers *.Cu *.Mask) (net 40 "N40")))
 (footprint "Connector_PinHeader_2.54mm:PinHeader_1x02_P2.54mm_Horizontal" (layer "B.Cu") (at 202.585 47.7975 90)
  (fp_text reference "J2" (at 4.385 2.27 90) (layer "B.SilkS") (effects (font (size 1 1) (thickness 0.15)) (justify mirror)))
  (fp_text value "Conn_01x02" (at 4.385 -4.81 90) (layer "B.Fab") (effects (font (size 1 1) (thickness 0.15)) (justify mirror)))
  (pad "1" thru_hole rect (at 0 0 90) (size 1.7 1.7) (drill 1) (layers *.Cu *.Mask) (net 43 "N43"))
  (pad "2" thru_hole oval (at 0 -2.54 90) (size 1.7 1.7) (drill 1) (layers *.Cu *.Mask) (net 42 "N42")))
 (gr_line (start 63.5 180.34) (end 63.5 43.18) (layer "Edge.Cuts") (width 0.1))
 (gr_line (start 243.84 180.34) (end 63.5 180.34) (layer "Edge.Cuts") (width 0.1))
 (gr_line (start 243.84 43.18) (end 243.84 180.34) (layer "Edge.Cuts") (width 0.1))
 (gr_line (start 63.5 43.18) (end 243.84 43.18) (layer "Edge.Cuts") (width 0.1))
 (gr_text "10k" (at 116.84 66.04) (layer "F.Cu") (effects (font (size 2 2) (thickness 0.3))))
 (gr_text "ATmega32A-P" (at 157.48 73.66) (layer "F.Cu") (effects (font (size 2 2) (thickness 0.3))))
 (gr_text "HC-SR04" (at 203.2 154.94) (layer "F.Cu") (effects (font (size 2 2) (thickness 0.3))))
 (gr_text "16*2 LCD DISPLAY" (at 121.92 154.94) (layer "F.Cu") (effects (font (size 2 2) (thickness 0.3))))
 (segment (start 132.08 106.68) (end 129.94798 104.54798) (width 0.25) (layer "F.Cu") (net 44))
 (segment (start 129.94798 60.55202) (end 137.16 53.34) (width 0.25) (layer "F.Cu") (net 44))
 (segment (start 129.94798 104.54798) (end 129.94798 60.55202) (width 0.25) (layer "F.Cu") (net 44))
 (segment (start 124.05202 104.54798) (end 121.92 106.68) (width 0.25) (layer "F.Cu") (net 44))
 (segment (start 129.94798 104.54798) (end 124.05202 104.54798) (width 0.25) (layer "F.Cu") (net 44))
 (segment (start 137.16 53.34) (end 137.16 47.555) (width 0.25) (layer "F.Cu") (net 44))
 (segment (start 124.46 106.68) (end 124.46 104.9975) (width 0.25) (layer "F.Cu") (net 40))
 (segment (start 124.46 107.43) (end 122.67 109.22) (width 0.25) (layer "F.Cu") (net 40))
 (segment (start 122.67 109.22) (end 111.76 109.22) (width 0.25) (layer "F.Cu") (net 40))
 (segment (start 124.46 106.68) (end 124.46 107.43) (width 0.25) (layer "F.Cu") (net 40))
 (segment (start 109.22 68.58) (end 130.245 47.555) (width 0.25) (layer "F.Cu") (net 40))
 (segment (start 130.245 47.555) (end 134.62 47.555) (width 0.25) (layer "F.Cu") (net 40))
 (segment (start 109.22 106.68) (end 109.22 73.66) (width 0.25) (layer "F.Cu") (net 40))
 (segment (start 111.76 109.22) (end 109.22 106.68) (width 0.25) (layer "F.Cu") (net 40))
 (segment (start 109.22 73.66) (end 109.22 68.58) (width 0.25) (layer "F.Cu") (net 40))
 (segment (start 202.585 47.7975) (end 202.585 52.725) (width 0.25) (layer "F.Cu") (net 43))
 (segment (start 202.585 52.725) (end 207.01 57.15) (width 0.25) (layer "F.Cu") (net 43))
 (segment (start 207.01 57.15) (end 207.01 130.575) (width 0.25) (layer "F.Cu") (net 43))
 (segment (start 203.435 134.62) (end 199.39 130.575) (width 0.25) (layer "F.Cu") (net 42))
 (segment (start 205.74 58.42) (end 205.74 134.62) (width 0.25) (layer "F.Cu") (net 42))
 (segment (start 205.74 134.62) (end 203.435 134.62) (width 0.25) (layer "F.Cu") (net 42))
 (segment (start 200.045 52.725) (end 205.74 58.42) (width 0.25) (layer "F.Cu") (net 42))
 (segment (start 200.045 47.7975) (end 200.045 52.725) (width 0.25) (layer "F.Cu") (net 42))
 (segment (start 116.84 86.36) (end 124.46 78.74) (width 0.25) (layer "F.Cu") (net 41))
 (segment (start 124.46 78.74) (end 124.46 73.66) (width 0.25) (layer "F.Cu") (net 41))
 (segment (start 116.84 106.68) (end 116.84 86.36) (width 0.25) (layer "F.Cu") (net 41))
 (segment (start 132.08 109.22) (end 133.30452 107.99548) (width 0.25) (layer "F.Cu") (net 14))
 (segment (start 129.54 106.68) (end 132.08 109.22) (width 0.25) (layer "F.Cu") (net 14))
 (segment (start 133.30452 107.99548) (end 133.30452 102.91548) (width 0.25) (layer "F.Cu") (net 14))
 (segment (start 133.30452 102.91548) (end 154.1275 82.0925) (width 0.25) (layer "F.Cu") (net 14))
 (segment (start 154.1275 82.0925) (end 171.395 82.0925) (width 0.25) (layer "F.Cu") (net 14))
 (segment (start 134.62 106.68) (end 134.62 104.14) (width 0.25) (layer "F.Cu") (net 15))
 (segment (start 134.62 104.14) (end 154.1275 84.6325) (width 0.25) (layer "F.Cu") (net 15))
 (segment (start 154.1275 84.6325) (end 171.395 84.6325) (width 0.25) (layer "F.Cu") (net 15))
 (segment (start 147.32 106.68) (end 161.7475 92.2525) (width 0.25) (layer "F.Cu") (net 18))
 (segment (start 161.7475 92.2525) (end 171.395 92.2525) (width 0.25) (layer "F.Cu") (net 18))
 (segment (start 161.7475 94.7925) (end 171.395 94.7925) (width 0.25) (layer "F.Cu") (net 19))
 (segment (start 149.86 106.68) (end 161.7475 94.7925) (width 0.25) (layer "F.Cu") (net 19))
 (segment (start 161.75512 97.3325) (end 171.395 97.3325) (width 0.25) (layer "F.Cu") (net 20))
 (segment (start 152.40508 106.68254) (end 161.75512 97.3325) (width 0.25) (layer "F.Cu") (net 20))
 (segment (start 154.94 106.68) (end 177.2875 106.68) (width 0.25) (layer "F.Cu") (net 21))
 (segment (start 177.2875 106.68) (end 186.635 97.3325) (width 0.25) (layer "F.Cu") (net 21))
 (segment (start 186.635 94.7925) (end 191.5475 94.7925) (width 0.25) (layer "F.Cu") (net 22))
 (segment (start 191.5475 94.7925) (end 201.93 105.175) (width 0.25) (layer "F.Cu") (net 22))
 (segment (start 201.93 105.175) (end 201.93 130.575) (width 0.25) (layer "F.Cu") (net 22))
 (segment (start 204.47 105.175) (end 204.47 130.575) (width 0.25) (layer "F.Cu") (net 23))
 (segment (start 186.635 92.2525) (end 191.5475 92.2525) (width 0.25) (layer "F.Cu") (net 23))
 (segment (start 191.5475 92.2525) (end 204.47 105.175) (width 0.25) (layer "F.Cu") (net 23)))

